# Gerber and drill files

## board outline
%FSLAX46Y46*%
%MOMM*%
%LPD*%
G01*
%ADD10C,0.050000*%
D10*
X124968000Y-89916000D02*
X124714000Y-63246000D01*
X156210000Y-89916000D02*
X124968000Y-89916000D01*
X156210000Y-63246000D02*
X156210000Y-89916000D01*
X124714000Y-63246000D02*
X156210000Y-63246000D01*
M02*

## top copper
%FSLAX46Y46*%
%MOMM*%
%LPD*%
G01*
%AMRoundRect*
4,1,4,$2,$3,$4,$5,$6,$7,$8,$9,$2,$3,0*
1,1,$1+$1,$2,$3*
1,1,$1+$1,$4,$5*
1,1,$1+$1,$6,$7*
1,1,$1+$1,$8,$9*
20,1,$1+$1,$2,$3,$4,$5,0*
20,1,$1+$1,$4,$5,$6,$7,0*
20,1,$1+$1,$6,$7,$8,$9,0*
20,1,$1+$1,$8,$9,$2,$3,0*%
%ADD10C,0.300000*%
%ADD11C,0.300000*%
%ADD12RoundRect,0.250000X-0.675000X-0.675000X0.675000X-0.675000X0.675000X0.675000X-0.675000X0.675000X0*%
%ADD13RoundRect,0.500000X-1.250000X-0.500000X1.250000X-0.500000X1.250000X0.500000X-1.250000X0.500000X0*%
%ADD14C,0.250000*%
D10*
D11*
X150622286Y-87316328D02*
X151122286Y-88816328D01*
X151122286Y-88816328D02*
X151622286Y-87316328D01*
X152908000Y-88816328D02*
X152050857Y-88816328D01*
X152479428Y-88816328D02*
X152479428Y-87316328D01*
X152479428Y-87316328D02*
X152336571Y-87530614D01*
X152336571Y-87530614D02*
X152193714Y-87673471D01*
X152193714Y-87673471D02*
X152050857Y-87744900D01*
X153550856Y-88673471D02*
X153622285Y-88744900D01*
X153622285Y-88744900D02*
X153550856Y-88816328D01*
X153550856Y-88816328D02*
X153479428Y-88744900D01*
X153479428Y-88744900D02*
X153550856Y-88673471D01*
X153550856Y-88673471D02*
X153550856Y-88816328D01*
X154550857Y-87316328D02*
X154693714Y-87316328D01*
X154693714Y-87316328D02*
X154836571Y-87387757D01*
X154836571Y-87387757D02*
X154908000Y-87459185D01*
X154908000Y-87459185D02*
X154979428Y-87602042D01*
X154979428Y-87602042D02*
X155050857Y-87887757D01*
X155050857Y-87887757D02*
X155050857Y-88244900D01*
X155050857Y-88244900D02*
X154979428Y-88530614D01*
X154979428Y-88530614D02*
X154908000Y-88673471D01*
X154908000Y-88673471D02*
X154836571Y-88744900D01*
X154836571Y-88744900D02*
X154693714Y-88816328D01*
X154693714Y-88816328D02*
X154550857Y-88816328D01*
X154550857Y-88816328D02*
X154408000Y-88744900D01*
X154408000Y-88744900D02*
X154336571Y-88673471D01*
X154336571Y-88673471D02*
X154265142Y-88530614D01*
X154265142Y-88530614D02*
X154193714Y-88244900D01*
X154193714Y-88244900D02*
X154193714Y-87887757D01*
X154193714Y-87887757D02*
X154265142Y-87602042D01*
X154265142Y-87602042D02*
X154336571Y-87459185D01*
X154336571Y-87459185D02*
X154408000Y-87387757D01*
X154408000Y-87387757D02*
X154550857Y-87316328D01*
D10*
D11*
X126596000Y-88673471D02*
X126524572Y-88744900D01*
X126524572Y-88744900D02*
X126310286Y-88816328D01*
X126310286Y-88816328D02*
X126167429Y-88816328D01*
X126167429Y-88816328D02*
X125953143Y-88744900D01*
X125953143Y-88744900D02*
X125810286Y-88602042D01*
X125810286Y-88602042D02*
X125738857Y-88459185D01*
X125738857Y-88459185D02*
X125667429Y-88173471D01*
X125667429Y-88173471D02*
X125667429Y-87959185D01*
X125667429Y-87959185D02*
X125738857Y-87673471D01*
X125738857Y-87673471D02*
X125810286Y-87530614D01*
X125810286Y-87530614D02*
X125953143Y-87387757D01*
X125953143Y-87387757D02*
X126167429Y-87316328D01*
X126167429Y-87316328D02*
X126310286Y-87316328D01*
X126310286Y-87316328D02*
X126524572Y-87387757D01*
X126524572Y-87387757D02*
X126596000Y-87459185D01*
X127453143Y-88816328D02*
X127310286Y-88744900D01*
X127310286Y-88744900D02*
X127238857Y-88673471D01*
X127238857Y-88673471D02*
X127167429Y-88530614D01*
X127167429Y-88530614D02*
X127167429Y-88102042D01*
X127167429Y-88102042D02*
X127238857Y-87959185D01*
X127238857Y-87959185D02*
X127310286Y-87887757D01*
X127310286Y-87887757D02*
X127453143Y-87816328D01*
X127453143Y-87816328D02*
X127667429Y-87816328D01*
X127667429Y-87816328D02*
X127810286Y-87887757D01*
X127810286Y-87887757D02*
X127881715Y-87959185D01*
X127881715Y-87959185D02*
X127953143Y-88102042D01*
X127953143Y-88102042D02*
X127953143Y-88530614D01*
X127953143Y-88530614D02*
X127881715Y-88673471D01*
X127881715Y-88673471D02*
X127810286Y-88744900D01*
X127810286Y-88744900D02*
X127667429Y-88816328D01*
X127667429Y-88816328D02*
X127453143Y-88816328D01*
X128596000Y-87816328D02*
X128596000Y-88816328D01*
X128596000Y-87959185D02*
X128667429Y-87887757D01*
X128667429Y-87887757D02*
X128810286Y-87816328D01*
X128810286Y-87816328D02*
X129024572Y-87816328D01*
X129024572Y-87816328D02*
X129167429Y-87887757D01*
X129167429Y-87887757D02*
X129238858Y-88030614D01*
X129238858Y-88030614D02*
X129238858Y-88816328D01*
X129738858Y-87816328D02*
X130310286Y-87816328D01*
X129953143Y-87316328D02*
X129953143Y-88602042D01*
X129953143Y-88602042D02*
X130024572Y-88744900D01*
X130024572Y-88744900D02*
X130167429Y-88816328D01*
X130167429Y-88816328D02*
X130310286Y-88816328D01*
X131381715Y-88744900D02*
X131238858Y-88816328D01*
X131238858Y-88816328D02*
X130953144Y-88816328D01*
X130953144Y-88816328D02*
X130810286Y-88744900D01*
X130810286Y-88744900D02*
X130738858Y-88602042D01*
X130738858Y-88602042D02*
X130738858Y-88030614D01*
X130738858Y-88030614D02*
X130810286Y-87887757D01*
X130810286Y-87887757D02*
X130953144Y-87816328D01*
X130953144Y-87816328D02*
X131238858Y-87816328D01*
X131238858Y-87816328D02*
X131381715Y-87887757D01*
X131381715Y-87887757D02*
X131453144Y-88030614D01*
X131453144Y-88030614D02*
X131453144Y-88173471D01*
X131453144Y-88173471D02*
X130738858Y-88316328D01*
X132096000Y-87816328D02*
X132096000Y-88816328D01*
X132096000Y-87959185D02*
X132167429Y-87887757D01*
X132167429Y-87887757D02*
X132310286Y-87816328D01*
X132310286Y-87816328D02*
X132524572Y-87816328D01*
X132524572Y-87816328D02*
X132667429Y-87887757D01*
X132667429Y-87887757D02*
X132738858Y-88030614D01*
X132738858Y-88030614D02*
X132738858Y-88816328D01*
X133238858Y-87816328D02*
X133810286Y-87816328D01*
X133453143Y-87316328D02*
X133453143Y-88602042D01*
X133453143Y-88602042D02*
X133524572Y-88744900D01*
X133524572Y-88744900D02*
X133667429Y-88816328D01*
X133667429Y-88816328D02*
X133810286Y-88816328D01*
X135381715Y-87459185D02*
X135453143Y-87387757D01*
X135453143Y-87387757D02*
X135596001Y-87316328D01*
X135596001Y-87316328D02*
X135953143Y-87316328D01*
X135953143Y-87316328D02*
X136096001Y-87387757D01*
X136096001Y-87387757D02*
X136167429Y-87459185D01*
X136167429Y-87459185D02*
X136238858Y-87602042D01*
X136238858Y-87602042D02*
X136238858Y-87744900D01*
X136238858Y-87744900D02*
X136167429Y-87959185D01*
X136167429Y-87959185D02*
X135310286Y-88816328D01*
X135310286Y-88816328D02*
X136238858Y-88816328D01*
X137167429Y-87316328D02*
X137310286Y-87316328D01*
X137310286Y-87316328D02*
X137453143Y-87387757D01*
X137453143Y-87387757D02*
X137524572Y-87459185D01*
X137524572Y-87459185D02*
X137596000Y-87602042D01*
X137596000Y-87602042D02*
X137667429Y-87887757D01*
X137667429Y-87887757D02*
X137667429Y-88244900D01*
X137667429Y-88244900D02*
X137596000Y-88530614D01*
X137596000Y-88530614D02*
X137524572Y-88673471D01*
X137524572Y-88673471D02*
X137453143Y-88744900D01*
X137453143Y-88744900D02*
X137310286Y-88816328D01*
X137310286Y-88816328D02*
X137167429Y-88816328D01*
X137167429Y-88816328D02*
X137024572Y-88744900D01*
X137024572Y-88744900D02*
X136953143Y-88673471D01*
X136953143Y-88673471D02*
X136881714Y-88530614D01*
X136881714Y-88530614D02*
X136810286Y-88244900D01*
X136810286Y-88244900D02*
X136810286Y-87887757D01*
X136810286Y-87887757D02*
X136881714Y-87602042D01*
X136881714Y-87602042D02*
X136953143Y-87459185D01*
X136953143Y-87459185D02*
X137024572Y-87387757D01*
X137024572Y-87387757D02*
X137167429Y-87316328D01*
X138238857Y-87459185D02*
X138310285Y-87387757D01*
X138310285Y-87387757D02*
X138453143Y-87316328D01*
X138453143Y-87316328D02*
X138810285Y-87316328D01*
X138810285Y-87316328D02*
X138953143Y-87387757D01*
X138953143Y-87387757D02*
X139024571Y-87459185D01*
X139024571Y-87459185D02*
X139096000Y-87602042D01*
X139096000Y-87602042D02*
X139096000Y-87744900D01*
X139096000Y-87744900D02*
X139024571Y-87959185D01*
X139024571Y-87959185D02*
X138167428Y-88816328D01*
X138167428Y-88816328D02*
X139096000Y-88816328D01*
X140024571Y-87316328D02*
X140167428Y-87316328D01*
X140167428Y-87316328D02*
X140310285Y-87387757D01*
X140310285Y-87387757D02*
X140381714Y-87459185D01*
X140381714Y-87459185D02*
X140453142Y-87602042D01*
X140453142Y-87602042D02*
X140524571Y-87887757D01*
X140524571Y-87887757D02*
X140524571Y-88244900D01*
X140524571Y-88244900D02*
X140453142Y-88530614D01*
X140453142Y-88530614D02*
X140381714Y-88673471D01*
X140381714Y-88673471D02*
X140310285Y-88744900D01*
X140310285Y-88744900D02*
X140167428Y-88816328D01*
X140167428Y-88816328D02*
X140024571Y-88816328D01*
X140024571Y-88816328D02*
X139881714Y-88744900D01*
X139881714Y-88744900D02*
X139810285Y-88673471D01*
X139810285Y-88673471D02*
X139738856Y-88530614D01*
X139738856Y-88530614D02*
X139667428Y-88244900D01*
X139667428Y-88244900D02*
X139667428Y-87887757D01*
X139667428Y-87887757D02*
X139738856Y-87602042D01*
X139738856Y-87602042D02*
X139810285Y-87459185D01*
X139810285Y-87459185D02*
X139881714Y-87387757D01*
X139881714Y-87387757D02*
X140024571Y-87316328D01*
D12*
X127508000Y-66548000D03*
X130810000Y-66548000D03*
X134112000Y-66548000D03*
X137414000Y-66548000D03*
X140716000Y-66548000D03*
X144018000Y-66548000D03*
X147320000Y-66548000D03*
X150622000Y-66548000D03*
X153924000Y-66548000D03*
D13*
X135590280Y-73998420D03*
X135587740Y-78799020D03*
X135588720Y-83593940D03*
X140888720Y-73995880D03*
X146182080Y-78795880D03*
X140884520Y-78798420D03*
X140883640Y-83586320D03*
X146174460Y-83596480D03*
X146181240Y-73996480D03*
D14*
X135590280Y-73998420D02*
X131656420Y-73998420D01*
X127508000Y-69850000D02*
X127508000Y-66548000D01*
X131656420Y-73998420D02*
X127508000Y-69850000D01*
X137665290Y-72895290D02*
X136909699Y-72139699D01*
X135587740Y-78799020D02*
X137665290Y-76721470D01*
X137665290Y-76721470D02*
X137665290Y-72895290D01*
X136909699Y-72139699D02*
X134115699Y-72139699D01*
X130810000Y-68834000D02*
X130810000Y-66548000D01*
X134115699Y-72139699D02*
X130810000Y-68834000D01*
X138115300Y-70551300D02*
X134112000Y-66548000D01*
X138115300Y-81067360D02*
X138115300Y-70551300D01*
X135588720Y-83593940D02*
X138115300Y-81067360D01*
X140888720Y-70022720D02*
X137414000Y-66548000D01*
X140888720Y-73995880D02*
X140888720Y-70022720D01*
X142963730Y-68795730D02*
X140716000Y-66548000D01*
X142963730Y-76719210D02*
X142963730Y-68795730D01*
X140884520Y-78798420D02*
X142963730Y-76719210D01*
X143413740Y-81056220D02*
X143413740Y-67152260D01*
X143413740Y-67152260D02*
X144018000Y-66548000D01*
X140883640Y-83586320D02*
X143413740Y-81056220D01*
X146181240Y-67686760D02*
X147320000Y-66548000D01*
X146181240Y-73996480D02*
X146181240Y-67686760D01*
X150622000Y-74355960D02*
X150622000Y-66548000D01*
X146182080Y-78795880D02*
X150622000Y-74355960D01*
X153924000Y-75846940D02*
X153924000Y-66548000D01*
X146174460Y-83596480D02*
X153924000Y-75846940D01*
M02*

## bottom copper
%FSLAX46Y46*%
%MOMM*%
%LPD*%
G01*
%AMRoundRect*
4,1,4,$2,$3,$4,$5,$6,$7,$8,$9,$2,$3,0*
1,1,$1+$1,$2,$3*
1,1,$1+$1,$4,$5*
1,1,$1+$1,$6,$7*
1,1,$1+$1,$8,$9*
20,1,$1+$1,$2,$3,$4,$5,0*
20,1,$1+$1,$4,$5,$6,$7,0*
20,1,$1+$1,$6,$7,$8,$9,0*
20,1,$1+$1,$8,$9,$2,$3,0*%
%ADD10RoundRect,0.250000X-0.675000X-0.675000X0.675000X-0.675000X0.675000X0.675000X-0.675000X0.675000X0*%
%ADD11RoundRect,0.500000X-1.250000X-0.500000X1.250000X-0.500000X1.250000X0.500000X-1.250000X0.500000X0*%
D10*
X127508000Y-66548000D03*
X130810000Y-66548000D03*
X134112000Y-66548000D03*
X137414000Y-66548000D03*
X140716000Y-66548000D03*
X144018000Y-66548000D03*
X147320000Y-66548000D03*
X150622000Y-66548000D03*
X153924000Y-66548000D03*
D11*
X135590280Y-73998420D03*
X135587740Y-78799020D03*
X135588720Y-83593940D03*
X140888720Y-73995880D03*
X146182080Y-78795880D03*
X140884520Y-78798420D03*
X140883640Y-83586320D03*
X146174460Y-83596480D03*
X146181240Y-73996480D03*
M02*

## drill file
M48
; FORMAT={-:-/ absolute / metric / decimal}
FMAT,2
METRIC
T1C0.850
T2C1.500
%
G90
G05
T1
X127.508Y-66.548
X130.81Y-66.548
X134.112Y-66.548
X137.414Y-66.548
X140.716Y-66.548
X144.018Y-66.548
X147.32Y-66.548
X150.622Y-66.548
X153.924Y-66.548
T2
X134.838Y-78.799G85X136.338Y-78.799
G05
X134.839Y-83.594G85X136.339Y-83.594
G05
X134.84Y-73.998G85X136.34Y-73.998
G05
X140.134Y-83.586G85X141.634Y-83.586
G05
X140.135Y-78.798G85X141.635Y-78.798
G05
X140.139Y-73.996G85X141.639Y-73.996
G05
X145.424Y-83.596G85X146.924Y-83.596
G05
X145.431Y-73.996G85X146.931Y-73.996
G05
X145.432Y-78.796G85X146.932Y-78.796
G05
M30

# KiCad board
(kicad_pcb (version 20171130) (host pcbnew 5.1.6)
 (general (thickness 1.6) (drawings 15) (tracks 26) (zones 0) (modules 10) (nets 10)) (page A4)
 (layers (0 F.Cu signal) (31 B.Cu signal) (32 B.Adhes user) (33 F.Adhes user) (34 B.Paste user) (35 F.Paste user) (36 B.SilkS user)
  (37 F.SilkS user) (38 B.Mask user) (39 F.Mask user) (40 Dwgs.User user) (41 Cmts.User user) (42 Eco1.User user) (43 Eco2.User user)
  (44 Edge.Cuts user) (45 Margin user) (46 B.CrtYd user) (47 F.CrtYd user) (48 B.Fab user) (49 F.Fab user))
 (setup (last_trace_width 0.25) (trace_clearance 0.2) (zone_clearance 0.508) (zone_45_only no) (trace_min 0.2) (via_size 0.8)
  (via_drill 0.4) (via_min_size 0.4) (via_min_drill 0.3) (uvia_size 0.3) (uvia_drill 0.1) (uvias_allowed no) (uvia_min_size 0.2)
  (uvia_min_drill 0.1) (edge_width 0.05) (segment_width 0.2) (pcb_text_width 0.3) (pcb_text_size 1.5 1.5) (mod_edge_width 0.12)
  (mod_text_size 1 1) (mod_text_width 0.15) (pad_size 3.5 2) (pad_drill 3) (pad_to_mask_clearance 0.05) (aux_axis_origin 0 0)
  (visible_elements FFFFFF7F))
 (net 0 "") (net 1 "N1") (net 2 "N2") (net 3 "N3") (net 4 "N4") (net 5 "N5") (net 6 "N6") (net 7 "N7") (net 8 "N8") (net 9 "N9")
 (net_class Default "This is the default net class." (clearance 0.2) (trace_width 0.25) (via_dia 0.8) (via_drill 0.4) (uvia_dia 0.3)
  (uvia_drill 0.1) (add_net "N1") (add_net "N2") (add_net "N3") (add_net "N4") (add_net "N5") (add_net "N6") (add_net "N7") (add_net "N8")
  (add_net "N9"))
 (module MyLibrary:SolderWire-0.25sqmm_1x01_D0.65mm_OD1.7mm (layer F.Cu) (at 127.508 66.548)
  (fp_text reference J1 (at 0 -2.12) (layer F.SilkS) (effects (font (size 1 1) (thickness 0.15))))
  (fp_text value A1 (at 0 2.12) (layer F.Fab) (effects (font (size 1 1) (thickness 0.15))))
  (pad 1 thru_hole roundrect (at 0 0) (size 1.85 1.85) (drill 0.85) (layers *.Cu *.Mask) (roundrect_rratio 0.135135) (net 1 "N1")))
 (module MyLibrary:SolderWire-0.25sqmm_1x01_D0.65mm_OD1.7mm (layer F.Cu) (at 130.81 66.548)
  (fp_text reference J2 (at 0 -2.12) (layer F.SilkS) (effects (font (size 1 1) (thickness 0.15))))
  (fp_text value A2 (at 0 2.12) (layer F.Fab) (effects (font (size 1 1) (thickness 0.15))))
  (pad 1 thru_hole roundrect (at 0 0) (size 1.85 1.85) (drill 0.85) (layers *.Cu *.Mask) (roundrect_rratio 0.135135) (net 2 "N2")))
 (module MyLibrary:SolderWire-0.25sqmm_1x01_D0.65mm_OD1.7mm (layer F.Cu) (at 134.112 66.548)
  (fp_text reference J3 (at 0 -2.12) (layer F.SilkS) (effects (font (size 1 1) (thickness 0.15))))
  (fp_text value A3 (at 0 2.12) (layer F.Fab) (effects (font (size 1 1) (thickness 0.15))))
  (pad 1 thru_hole roundrect (at 0 0) (size 1.85 1.85) (drill 0.85) (layers *.Cu *.Mask) (roundrect_rratio 0.135135) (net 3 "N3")))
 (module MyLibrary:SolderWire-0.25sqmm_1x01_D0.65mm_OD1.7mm (layer F.Cu) (at 137.414 66.548)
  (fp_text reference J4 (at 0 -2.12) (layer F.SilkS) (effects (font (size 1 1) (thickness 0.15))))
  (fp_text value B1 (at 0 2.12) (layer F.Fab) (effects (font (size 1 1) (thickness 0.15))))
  (pad 1 thru_hole roundrect (at 0 0) (size 1.85 1.85) (drill 0.85) (layers *.Cu *.Mask) (roundrect_rratio 0.135135) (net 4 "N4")))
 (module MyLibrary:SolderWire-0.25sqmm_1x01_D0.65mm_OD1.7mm (layer F.Cu) (at 140.716 66.548)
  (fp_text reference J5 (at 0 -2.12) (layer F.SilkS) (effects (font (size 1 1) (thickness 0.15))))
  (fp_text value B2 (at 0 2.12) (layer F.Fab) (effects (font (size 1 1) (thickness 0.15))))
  (pad 1 thru_hole roundrect (at 0 0) (size 1.85 1.85) (drill 0.85) (layers *.Cu *.Mask) (roundrect_rratio 0.135135) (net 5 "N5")))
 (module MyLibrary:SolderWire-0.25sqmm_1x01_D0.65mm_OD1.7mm (layer F.Cu) (at 144.018 66.548)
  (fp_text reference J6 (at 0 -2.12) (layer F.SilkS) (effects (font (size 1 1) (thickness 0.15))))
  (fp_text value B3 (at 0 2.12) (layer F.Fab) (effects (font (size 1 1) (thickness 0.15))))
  (pad 1 thru_hole roundrect (at 0 0) (size 1.85 1.85) (drill 0.85) (layers *.Cu *.Mask) (roundrect_rratio 0.135135) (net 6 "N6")))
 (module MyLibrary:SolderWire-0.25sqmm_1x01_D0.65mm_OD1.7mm (layer F.Cu) (at 147.32 66.548)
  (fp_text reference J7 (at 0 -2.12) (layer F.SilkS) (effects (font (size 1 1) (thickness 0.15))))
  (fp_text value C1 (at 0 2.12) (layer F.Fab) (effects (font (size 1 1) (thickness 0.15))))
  (pad 1 thru_hole roundrect (at 0 0) (size 1.85 1.85) (drill 0.85) (layers *.Cu *.Mask) (roundrect_rratio 0.135135) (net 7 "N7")))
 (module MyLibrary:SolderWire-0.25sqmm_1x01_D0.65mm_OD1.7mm (layer F.Cu) (at 150.622 66.548)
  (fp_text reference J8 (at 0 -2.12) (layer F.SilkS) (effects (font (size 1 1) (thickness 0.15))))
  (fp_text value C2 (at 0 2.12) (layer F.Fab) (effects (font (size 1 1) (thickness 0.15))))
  (pad 1 thru_hole roundrect (at 0 0) (size 1.85 1.85) (drill 0.85) (layers *.Cu *.Mask) (roundrect_rratio 0.135135) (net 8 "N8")))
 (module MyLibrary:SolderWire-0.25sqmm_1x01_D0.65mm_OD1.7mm (layer F.Cu) (at 153.924 66.548)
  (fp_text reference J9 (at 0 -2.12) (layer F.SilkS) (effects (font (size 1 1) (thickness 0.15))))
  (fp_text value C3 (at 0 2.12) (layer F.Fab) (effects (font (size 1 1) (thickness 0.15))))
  (pad 1 thru_hole roundrect (at 0 0) (size 1.85 1.85) (drill 0.85) (layers *.Cu *.Mask) (roundrect_rratio 0.135135) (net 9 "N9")))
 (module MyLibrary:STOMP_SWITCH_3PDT (layer F.Cu) (at 140.97 78.74)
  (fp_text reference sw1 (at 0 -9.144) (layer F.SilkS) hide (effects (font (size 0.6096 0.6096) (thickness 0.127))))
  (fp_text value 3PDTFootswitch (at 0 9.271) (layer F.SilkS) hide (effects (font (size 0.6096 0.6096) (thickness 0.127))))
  (pad A1 thru_hole roundrect (at -5.37972 -4.74158) (size 3.5 2) (drill oval 3 1.5) (layers *.Cu *.Mask) (roundrect_rratio 0.25)
   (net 1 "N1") (solder_mask_margin 0.1016))
  (pad A2 thru_hole roundrect (at -5.38226 0.05902) (size 3.5 2) (drill oval 3 1.5) (layers *.Cu *.Mask) (roundrect_rratio 0.25)
   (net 2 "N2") (solder_mask_margin 0.1016))
  (pad A3 thru_hole roundrect (at -5.38128 4.85394) (size 3.5 2) (drill oval 3 1.5) (layers *.Cu *.Mask) (roundrect_rratio 0.25)
   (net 3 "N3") (solder_mask_margin 0.1016))
  (pad B1 thru_hole roundrect (at -0.08128 -4.74412) (size 3.5 2) (drill oval 3 1.5) (layers *.Cu *.Mask) (roundrect_rratio 0.25)
   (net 4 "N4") (solder_mask_margin 0.1016))
  (pad C2 thru_hole roundrect (at 5.21208 0.05588) (size 3.5 2) (drill oval 3 1.5) (layers *.Cu *.Mask) (roundrect_rratio 0.25) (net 8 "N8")
   (solder_mask_margin 0.1016))
  (pad B2 thru_hole roundrect (at -0.08548 0.05842) (size 3.5 2) (drill oval 3 1.5) (layers *.Cu *.Mask) (roundrect_rratio 0.25)
   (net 5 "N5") (solder_mask_margin 0.1016))
  (pad B3 thru_hole roundrect (at -0.08636 4.84632) (size 3.5 2) (drill oval 3 1.5) (layers *.Cu *.Mask) (roundrect_rratio 0.25)
   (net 6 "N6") (solder_mask_margin 0.1016))
  (pad C3 thru_hole roundrect (at 5.20446 4.85648) (size 3.5 2) (drill oval 3 1.5) (layers *.Cu *.Mask) (roundrect_rratio 0.25) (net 9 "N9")
   (solder_mask_margin 0.1016))
  (pad C1 thru_hole roundrect (at 5.21124 -4.74352) (size 3.5 2) (drill oval 3 1.5) (layers *.Cu *.Mask) (roundrect_rratio 0.25)
   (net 7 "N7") (solder_mask_margin 0.1016)))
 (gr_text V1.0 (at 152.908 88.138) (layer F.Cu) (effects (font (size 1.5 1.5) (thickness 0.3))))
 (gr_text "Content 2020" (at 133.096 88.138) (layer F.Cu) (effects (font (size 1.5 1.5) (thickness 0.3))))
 (gr_line (start 124.968 89.916) (end 124.714 63.246) (layer Edge.Cuts) (width 0.05))
 (gr_line (start 156.21 89.916) (end 124.968 89.916) (layer Edge.Cuts) (width 0.05))
 (gr_line (start 156.21 63.246) (end 156.21 89.916) (layer Edge.Cuts) (width 0.05))
 (gr_line (start 124.714 63.246) (end 156.21 63.246) (layer Edge.Cuts) (width 0.05))
 (segment (start 135.59028 73.99842) (end 131.65642 73.99842) (width 0.25) (layer F.Cu) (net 1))
 (segment (start 127.508 69.85) (end 127.508 66.548) (width 0.25) (layer F.Cu) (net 1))
 (segment (start 131.65642 73.99842) (end 127.508 69.85) (width 0.25) (layer F.Cu) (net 1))
 (segment (start 137.66529 72.89529) (end 136.909699 72.139699) (width 0.25) (layer F.Cu) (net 2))
 (segment (start 135.58774 78.79902) (end 137.66529 76.72147) (width 0.25) (layer F.Cu) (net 2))
 (segment (start 137.66529 76.72147) (end 137.66529 72.89529) (width 0.25) (layer F.Cu) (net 2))
 (segment (start 136.909699 72.139699) (end 134.115699 72.139699) (width 0.25) (layer F.Cu) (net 2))
 (segment (start 130.81 68.834) (end 130.81 66.548) (width 0.25) (layer F.Cu) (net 2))
 (segment (start 134.115699 72.139699) (end 130.81 68.834) (width 0.25) (layer F.Cu) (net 2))
 (segment (start 138.1153 70.5513) (end 134.112 66.548) (width 0.25) (layer F.Cu) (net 3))
 (segment (start 138.1153 81.06736) (end 138.1153 70.5513) (width 0.25) (layer F.Cu) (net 3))
 (segment (start 135.58872 83.59394) (end 138.1153 81.06736) (width 0.25) (layer F.Cu) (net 3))
 (segment (start 140.88872 70.02272) (end 137.414 66.548) (width 0.25) (layer F.Cu) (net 4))
 (segment (start 140.88872 73.99588) (end 140.88872 70.02272) (width 0.25) (layer F.Cu) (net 4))
 (segment (start 142.96373 68.79573) (end 140.716 66.548) (width 0.25) (layer F.Cu) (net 5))
 (segment (start 142.96373 76.71921) (end 142.96373 68.79573) (width 0.25) (layer F.Cu) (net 5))
 (segment (start 140.88452 78.79842) (end 142.96373 76.71921) (width 0.25) (layer F.Cu) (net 5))
 (segment (start 143.41374 81.05622) (end 143.41374 67.15226) (width 0.25) (layer F.Cu) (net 6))
 (segment (start 143.41374 67.15226) (end 144.018 66.548) (width 0.25) (layer F.Cu) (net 6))
 (segment (start 140.88364 83.58632) (end 143.41374 81.05622) (width 0.25) (layer F.Cu) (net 6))
 (segment (start 146.18124 67.68676) (end 147.32 66.548) (width 0.25) (layer F.Cu) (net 7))
 (segment (start 146.18124 73.99648) (end 146.18124 67.68676) (width 0.25) (layer F.Cu) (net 7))
 (segment (start 150.622 74.35596) (end 150.622 66.548) (width 0.25) (layer F.Cu) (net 8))
 (segment (start 146.18208 78.79588) (end 150.622 74.35596) (width 0.25) (layer F.Cu) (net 8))
 (segment (start 153.924 75.84694) (end 153.924 66.548) (width 0.25) (layer F.Cu) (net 9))
 (segment (start 146.17446 83.59648) (end 153.924 75.84694) (width 0.25) (layer F.Cu) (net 9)))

